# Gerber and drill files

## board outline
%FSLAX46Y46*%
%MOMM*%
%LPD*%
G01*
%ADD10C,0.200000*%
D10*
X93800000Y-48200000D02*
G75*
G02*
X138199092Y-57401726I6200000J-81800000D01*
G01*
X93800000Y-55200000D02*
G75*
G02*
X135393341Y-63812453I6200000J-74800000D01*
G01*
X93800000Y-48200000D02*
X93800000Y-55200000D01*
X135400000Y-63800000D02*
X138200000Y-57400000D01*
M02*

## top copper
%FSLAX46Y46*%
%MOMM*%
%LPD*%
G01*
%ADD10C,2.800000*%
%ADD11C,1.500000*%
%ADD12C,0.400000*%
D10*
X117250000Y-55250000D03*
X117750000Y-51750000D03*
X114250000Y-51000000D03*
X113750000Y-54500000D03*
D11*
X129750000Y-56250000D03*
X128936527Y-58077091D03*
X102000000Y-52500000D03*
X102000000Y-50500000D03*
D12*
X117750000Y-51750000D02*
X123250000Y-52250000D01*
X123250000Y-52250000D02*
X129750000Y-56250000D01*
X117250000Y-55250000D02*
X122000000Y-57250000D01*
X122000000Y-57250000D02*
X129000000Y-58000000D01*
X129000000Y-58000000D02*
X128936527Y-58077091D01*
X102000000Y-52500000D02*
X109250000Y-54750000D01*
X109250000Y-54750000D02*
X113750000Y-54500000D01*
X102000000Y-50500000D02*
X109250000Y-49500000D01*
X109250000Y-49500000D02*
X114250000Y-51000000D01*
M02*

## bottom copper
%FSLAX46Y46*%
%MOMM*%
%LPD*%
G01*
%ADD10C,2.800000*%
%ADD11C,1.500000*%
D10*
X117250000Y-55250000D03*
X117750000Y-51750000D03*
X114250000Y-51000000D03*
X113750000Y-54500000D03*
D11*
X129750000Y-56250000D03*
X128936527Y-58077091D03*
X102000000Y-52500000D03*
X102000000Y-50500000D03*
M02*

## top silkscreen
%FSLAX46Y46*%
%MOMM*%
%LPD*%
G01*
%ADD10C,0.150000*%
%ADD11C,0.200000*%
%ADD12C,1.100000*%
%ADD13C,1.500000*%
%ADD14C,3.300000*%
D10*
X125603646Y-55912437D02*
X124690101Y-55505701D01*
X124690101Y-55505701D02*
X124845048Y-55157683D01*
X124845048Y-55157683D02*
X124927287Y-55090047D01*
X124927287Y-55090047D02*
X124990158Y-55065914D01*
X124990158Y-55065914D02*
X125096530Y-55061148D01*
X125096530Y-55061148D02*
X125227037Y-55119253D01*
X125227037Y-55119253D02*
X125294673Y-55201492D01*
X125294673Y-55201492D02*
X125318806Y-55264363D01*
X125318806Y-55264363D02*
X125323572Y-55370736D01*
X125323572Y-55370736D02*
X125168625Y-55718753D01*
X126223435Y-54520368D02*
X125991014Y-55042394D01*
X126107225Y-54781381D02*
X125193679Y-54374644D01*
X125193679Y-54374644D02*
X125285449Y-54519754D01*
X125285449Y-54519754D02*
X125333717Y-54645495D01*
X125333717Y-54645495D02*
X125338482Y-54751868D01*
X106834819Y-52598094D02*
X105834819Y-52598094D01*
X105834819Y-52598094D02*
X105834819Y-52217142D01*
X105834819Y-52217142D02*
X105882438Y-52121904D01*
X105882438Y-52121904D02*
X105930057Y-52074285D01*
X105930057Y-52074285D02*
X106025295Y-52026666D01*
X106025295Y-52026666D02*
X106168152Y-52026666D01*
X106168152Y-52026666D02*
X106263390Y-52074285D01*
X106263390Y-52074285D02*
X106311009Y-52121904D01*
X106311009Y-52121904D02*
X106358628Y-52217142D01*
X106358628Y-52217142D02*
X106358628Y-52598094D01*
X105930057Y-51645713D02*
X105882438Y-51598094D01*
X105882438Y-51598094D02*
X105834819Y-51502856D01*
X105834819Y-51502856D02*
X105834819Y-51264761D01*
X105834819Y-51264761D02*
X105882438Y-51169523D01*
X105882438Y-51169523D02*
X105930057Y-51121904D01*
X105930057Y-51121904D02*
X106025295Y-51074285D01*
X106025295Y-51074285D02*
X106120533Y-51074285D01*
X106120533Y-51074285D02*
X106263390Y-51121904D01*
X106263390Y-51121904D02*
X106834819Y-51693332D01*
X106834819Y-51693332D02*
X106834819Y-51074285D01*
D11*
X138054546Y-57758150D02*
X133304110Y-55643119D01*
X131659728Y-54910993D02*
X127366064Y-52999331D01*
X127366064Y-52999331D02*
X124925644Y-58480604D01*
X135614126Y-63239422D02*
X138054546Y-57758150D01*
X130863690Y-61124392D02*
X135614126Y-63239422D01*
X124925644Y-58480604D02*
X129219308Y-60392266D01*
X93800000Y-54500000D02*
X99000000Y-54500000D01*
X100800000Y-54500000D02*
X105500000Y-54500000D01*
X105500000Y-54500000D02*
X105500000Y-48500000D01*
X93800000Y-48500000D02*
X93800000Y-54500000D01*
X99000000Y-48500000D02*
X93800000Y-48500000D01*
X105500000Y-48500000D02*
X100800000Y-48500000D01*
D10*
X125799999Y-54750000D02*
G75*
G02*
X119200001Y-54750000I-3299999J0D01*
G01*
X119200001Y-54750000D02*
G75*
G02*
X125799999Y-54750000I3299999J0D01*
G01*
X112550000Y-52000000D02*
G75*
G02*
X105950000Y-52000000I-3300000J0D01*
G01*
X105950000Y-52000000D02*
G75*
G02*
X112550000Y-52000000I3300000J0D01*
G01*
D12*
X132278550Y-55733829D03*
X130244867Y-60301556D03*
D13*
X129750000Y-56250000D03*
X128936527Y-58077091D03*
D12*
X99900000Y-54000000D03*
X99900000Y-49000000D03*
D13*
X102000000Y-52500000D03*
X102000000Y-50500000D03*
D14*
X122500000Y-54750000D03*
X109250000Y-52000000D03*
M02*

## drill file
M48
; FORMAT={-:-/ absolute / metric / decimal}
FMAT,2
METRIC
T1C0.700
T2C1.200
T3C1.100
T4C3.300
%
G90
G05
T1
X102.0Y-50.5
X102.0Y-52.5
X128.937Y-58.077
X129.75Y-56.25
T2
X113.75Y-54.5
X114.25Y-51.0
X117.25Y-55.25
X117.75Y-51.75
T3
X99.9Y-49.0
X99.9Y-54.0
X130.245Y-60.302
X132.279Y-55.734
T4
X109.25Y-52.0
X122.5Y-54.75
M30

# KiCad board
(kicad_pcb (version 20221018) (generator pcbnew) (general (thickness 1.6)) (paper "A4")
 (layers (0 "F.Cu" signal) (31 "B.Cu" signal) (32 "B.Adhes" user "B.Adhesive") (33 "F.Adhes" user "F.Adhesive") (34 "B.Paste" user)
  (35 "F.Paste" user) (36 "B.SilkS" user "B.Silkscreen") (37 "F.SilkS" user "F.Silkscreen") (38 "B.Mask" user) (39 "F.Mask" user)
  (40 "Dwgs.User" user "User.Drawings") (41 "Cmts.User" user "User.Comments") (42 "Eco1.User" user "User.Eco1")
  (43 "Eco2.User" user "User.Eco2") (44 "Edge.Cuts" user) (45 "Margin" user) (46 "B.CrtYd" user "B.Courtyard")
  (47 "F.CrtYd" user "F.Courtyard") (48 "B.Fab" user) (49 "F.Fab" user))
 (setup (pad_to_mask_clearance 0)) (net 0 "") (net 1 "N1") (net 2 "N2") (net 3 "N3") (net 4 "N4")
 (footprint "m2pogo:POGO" (layer "F.Cu") (at 117.25 55.25)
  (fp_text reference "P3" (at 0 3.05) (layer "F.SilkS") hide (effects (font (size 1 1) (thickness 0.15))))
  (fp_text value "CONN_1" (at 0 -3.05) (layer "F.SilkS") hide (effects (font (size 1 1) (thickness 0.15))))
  (pad "1" thru_hole circle (at 0 0) (size 2.8 2.8) (drill 1.2) (layers "*.Cu" "*.Mask") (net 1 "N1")))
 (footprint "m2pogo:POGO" (layer "F.Cu") (at 117.75 51.75)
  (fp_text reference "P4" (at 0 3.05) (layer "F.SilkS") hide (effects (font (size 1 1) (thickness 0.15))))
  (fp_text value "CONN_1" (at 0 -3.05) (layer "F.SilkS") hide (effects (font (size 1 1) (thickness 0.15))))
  (pad "1" thru_hole circle (at 0 0) (size 2.8 2.8) (drill 1.2) (layers "*.Cu" "*.Mask") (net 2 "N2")))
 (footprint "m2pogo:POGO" (layer "F.Cu") (at 114.25 51)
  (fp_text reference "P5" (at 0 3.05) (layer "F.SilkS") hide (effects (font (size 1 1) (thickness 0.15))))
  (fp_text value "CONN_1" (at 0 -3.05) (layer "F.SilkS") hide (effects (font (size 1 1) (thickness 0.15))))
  (pad "1" thru_hole circle (at 0 0) (size 2.8 2.8) (drill 1.2) (layers "*.Cu" "*.Mask") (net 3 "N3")))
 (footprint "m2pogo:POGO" (layer "F.Cu") (at 113.75 54.5)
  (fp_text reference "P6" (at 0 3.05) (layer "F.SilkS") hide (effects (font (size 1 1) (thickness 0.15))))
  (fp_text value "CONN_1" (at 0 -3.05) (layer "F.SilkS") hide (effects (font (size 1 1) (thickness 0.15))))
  (pad "1" thru_hole circle (at 0 0) (size 2.8 2.8) (drill 1.2) (layers "*.Cu" "*.Mask") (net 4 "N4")))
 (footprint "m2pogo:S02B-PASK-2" (layer "F.Cu") (at 129.75 56.25 -114)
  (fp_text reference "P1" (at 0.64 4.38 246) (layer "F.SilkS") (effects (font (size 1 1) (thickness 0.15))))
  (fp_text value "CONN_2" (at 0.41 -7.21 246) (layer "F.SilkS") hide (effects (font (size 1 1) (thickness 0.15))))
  (fp_line (start -2 -8.2) (end -2 -3) (stroke (width 0.2) (type solid)) (layer "F.SilkS"))
  (fp_line (start -2 -1.2) (end -2 3.5) (stroke (width 0.2) (type solid)) (layer "F.SilkS"))
  (fp_line (start -2 3.5) (end 4 3.5) (stroke (width 0.2) (type solid)) (layer "F.SilkS"))
  (fp_line (start 4 -8.2) (end -2 -8.2) (stroke (width 0.2) (type solid)) (layer "F.SilkS"))
  (fp_line (start 4 -3) (end 4 -8.2) (stroke (width 0.2) (type solid)) (layer "F.SilkS"))
  (fp_line (start 4 3.5) (end 4 -1.2) (stroke (width 0.2) (type solid)) (layer "F.SilkS"))
  (pad "" np_thru_hole circle (at -1.5 -2.1 246) (size 1.1 1.1) (drill 1.1) (layers "*.Cu" "*.Mask" "F.SilkS"))
  (pad "" np_thru_hole circle (at 3.5 -2.1 246) (size 1.1 1.1) (drill 1.1) (layers "*.Cu" "*.Mask" "F.SilkS"))
  (pad "1" thru_hole circle (at 0 0 246) (size 1.5 1.5) (drill 0.7) (layers "*.Cu" "*.Mask" "F.SilkS") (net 2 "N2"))
  (pad "2" thru_hole circle (at 2 0 246) (size 1.5 1.5) (drill 0.7) (layers "*.Cu" "*.Mask" "F.SilkS") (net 1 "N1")))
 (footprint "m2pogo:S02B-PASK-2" (layer "F.Cu") (at 102 52.5 90)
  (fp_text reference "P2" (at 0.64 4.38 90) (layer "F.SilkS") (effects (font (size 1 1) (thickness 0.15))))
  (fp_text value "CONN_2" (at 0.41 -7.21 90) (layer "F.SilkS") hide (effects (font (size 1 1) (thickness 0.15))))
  (fp_line (start -2 -8.2) (end -2 -3) (stroke (width 0.2) (type solid)) (layer "F.SilkS"))
  (fp_line (start -2 -1.2) (end -2 3.5) (stroke (width 0.2) (type solid)) (layer "F.SilkS"))
  (fp_line (start -2 3.5) (end 4 3.5) (stroke (width 0.2) (type solid)) (layer "F.SilkS"))
  (fp_line (start 4 -8.2) (end -2 -8.2) (stroke (width 0.2) (type solid)) (layer "F.SilkS"))
  (fp_line (start 4 -3) (end 4 -8.2) (stroke (width 0.2) (type solid)) (layer "F.SilkS"))
  (fp_line (start 4 3.5) (end 4 -1.2) (stroke (width 0.2) (type solid)) (layer "F.SilkS"))
  (pad "" np_thru_hole circle (at -1.5 -2.1 90) (size 1.1 1.1) (drill 1.1) (layers "*.Cu" "*.Mask" "F.SilkS"))
  (pad "" np_thru_hole circle (at 3.5 -2.1 90) (size 1.1 1.1) (drill 1.1) (layers "*.Cu" "*.Mask" "F.SilkS"))
  (pad "1" thru_hole circle (at 0 0 90) (size 1.5 1.5) (drill 0.7) (layers "*.Cu" "*.Mask" "F.SilkS") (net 4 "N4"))
  (pad "2" thru_hole circle (at 2 0 90) (size 1.5 1.5) (drill 0.7) (layers "*.Cu" "*.Mask" "F.SilkS") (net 3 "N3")))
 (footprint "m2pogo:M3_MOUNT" (layer "F.Cu") (at 122.5 54.75 67.5)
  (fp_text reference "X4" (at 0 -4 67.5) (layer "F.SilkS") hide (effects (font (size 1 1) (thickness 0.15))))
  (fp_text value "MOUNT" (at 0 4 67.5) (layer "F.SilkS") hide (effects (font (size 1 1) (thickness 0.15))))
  (fp_circle (center 0 0) (end 3.3 0) (stroke (width 0.15) (type solid)) (fill none) (layer "F.SilkS"))
  (pad "" np_thru_hole circle (at 0 0 67.5) (size 3.3 3.3) (drill 3.3) (layers "*.Cu" "*.Mask" "F.Paste" "F.SilkS")))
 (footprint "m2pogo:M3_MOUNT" (layer "F.Cu") (at 109.25 52)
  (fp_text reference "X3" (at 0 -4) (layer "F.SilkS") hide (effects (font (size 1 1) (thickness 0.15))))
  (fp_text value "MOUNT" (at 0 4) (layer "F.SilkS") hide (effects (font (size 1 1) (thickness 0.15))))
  (fp_circle (center 0 0) (end 3.3 0) (stroke (width 0.15) (type solid)) (fill none) (layer "F.SilkS"))
  (pad "" np_thru_hole circle (at 0 0) (size 3.3 3.3) (drill 3.3) (layers "*.Cu" "*.Mask" "F.Paste" "F.SilkS")))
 (gr_arc (start 93.8 48.2) (mid 116.647925 49.67238) (end 138.199092 57.401726) (stroke (width 0.2) (type solid)) (layer "Edge.Cuts"))
 (gr_arc (start 93.8 55.2) (mid 115.218619 56.50256) (end 135.393341 63.812453) (stroke (width 0.2) (type solid)) (layer "Edge.Cuts"))
 (gr_line (start 93.8 48.2) (end 93.8 55.2) (stroke (width 0.2) (type solid)) (layer "Edge.Cuts"))
 (gr_line (start 135.4 63.8) (end 138.2 57.4) (stroke (width 0.2) (type solid)) (layer "Edge.Cuts"))
 (segment (start 117.75 51.75) (end 123.25 52.25) (width 0.4) (layer "F.Cu") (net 2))
 (segment (start 123.25 52.25) (end 129.75 56.25) (width 0.4) (layer "F.Cu") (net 2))
 (segment (start 117.25 55.25) (end 122 57.25) (width 0.4) (layer "F.Cu") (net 1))
 (segment (start 122 57.25) (end 129 58) (width 0.4) (layer "F.Cu") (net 1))
 (segment (start 129 58) (end 128.936527 58.077091) (width 0.4) (layer "F.Cu") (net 1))
 (segment (start 102 52.5) (end 109.25 54.75) (width 0.4) (layer "F.Cu") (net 4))
 (segment (start 109.25 54.75) (end 113.75 54.5) (width 0.4) (layer "F.Cu") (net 4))
 (segment (start 102 50.5) (end 109.25 49.5) (width 0.4) (layer "F.Cu") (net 3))
 (segment (start 109.25 49.5) (end 114.25 51) (width 0.4) (layer "F.Cu") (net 3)))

